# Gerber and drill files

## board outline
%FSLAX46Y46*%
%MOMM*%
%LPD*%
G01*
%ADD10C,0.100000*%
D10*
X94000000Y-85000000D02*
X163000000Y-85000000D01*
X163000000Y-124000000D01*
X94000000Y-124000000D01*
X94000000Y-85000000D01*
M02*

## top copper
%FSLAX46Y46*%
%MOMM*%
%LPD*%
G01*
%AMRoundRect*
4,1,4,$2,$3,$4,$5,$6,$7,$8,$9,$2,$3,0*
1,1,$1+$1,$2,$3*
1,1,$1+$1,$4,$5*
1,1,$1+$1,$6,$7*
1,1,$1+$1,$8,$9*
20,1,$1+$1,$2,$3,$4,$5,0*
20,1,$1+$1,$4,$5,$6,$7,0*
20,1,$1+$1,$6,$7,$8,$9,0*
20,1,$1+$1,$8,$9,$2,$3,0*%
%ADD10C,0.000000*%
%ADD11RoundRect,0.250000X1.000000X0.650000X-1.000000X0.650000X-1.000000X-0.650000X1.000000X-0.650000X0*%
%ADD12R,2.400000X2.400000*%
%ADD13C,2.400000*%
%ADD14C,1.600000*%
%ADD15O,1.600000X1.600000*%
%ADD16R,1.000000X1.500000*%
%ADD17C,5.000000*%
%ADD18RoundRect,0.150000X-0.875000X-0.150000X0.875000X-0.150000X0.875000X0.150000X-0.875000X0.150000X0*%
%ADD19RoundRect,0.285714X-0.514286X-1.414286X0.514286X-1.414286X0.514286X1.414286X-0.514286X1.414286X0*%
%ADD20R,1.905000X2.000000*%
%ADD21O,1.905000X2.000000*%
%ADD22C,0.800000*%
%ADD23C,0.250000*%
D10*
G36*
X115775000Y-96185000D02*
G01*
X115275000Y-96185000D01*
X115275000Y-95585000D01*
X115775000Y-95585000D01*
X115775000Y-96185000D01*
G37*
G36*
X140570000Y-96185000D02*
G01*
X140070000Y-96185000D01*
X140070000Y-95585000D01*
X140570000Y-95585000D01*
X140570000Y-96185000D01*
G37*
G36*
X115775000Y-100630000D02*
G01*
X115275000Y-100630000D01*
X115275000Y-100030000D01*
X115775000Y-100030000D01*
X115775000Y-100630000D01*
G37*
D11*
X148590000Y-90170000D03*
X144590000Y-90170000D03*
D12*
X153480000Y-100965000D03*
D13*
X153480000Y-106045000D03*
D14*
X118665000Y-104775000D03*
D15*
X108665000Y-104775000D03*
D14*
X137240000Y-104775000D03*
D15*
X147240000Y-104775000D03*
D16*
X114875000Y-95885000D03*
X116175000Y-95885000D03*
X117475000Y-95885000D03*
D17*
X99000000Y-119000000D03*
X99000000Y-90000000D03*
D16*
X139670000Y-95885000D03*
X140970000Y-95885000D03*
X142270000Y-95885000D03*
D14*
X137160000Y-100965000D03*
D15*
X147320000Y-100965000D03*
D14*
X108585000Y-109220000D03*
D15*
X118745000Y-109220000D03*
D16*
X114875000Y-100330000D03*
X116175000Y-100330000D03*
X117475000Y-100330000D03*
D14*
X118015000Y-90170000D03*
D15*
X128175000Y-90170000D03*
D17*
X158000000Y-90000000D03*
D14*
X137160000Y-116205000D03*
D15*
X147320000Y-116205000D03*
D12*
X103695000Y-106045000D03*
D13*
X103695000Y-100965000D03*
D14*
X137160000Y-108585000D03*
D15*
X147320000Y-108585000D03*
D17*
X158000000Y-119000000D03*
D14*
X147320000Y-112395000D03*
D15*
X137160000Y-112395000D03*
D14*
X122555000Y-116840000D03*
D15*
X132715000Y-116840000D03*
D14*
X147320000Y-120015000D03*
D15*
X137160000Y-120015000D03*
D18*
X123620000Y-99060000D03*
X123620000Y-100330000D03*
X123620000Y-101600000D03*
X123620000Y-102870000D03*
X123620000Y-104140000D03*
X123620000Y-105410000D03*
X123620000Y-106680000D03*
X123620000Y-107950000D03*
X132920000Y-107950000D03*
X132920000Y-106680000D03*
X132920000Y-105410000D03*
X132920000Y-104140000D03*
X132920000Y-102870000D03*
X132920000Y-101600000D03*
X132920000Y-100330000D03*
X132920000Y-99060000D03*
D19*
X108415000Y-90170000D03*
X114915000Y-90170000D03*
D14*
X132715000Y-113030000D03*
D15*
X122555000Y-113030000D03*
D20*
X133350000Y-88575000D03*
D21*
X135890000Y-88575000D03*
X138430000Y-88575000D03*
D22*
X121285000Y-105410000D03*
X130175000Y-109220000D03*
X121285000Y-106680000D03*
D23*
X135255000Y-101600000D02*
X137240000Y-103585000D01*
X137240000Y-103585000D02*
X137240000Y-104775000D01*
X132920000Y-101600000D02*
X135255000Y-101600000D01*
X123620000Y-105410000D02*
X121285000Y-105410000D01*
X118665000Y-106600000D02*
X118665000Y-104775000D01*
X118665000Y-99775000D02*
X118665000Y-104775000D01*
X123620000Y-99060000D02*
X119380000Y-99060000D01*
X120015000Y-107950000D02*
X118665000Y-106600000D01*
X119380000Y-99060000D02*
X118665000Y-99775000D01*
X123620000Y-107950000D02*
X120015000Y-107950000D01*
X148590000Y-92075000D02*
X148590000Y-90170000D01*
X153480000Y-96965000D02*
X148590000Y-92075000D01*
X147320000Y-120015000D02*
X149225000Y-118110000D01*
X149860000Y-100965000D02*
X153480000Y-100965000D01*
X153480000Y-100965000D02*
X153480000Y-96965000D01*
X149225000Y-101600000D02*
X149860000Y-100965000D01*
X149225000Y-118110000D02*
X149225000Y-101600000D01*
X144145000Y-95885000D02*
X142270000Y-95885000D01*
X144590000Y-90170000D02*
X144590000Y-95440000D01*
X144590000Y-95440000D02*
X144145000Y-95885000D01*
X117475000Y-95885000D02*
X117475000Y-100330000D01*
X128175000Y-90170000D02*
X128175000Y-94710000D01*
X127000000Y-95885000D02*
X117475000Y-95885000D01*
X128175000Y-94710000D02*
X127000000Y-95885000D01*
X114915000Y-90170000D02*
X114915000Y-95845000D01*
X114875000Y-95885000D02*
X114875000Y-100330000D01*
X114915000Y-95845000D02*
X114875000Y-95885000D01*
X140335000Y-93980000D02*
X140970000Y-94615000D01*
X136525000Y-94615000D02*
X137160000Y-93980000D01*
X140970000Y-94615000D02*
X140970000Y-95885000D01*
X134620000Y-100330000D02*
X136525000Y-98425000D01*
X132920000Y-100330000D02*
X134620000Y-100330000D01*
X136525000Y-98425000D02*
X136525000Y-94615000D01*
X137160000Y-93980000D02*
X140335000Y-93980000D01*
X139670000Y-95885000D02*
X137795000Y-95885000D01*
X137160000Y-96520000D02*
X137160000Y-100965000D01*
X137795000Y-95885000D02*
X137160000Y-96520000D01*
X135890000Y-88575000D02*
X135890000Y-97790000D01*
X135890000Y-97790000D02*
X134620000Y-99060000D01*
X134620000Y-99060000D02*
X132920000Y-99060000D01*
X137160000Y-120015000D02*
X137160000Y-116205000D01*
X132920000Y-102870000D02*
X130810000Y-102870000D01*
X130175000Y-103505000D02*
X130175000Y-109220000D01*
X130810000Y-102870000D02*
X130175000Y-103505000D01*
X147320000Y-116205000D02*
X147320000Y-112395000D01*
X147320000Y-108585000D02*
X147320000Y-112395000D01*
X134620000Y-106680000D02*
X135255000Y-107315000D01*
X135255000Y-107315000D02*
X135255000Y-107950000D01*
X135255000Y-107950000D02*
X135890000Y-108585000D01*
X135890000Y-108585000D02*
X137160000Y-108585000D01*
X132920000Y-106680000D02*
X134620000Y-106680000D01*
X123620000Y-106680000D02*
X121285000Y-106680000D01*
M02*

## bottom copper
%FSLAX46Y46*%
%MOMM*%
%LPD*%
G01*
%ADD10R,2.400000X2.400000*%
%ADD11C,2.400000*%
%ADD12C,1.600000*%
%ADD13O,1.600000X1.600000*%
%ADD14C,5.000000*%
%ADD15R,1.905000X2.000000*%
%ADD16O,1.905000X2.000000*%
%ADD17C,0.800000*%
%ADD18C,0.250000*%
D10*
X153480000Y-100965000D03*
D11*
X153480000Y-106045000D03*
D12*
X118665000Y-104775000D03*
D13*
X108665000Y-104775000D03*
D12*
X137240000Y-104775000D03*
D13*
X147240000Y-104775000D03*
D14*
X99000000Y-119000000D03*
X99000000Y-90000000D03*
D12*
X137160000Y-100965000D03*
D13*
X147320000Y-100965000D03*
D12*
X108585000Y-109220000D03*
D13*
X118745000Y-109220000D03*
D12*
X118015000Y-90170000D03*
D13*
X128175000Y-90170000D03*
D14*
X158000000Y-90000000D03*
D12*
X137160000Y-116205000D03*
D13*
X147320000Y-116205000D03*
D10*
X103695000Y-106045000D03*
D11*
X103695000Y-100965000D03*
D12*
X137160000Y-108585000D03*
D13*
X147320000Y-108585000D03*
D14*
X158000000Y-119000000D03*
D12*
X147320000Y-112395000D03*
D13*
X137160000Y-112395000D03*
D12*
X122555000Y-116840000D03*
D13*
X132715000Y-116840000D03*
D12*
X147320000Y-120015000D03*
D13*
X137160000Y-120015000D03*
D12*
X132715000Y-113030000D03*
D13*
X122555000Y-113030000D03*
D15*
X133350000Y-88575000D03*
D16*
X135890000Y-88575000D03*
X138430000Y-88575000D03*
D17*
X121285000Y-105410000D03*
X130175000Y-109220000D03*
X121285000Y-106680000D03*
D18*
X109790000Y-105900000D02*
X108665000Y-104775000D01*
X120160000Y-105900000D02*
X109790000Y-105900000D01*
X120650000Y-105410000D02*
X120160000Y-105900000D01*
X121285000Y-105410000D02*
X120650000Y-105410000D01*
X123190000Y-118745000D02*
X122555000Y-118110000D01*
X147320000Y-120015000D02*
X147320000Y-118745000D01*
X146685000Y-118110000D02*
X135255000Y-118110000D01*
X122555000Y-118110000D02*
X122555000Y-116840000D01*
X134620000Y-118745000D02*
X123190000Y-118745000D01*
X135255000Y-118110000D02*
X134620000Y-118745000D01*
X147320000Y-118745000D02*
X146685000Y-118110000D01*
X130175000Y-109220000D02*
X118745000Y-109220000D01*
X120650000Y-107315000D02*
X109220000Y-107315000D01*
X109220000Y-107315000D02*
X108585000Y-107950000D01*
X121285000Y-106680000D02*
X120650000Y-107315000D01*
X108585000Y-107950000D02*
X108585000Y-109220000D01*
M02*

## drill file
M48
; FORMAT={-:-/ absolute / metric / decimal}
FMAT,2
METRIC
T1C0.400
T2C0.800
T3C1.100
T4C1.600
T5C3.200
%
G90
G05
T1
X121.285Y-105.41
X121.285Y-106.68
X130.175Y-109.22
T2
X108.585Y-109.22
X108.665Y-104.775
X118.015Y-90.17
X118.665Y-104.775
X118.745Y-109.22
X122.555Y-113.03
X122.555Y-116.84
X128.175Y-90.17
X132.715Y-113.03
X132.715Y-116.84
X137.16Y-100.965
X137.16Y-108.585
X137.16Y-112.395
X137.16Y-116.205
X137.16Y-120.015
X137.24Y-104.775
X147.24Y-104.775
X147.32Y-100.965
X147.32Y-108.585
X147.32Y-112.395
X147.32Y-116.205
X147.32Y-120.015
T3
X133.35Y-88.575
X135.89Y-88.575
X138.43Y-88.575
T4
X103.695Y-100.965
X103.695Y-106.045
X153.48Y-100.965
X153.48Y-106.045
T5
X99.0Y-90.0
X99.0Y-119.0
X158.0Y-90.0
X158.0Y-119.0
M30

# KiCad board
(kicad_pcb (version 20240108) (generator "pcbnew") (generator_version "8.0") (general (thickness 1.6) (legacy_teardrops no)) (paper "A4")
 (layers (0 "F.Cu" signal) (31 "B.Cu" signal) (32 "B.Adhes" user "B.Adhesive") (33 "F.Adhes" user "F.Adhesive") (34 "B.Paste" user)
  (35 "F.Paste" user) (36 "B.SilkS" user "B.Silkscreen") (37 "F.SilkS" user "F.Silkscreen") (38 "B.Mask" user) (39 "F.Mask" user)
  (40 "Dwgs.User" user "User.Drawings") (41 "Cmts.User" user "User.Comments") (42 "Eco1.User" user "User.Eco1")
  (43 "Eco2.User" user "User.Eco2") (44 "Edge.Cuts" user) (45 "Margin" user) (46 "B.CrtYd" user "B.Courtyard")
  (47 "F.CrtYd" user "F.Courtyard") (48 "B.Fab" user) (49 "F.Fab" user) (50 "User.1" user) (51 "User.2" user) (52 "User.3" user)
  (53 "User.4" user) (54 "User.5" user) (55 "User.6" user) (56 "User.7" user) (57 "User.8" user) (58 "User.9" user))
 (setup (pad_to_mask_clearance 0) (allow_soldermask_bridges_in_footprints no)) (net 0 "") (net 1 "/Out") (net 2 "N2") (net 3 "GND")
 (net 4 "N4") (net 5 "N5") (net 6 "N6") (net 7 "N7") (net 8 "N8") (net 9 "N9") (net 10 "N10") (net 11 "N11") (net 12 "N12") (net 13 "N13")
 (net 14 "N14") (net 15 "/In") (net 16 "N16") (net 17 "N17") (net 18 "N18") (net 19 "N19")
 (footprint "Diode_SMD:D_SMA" (layer "F.Cu") (at 146.59 90.17 180)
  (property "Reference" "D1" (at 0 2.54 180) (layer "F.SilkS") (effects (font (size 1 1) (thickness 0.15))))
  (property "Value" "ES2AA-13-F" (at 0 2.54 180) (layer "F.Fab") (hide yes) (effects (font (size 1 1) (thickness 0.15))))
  (pad "1" smd roundrect (at -2 0 180) (size 2.5 1.8) (layers "F.Cu" "F.Paste" "F.Mask") (roundrect_rratio 0.1388888889) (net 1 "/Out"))
  (pad "2" smd roundrect (at 2 0 180) (size 2.5 1.8) (layers "F.Cu" "F.Paste" "F.Mask") (roundrect_rratio 0.1388888889) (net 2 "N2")))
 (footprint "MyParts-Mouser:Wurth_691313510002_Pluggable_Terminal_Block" (layer "F.Cu") (at 153.48 100.965 -90)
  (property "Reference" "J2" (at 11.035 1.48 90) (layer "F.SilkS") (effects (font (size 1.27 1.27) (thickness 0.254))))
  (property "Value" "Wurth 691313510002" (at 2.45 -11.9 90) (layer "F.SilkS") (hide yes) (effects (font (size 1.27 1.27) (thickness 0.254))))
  (pad "1" thru_hole rect (at 0 0 270) (size 2.4 2.4) (drill 1.6) (layers "*.Cu" "*.Mask") (remove_unused_layers no) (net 1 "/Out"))
  (pad "2" thru_hole circle (at 5.08 0 270) (size 2.4 2.4) (drill 1.6) (layers "*.Cu" "*.Mask") (remove_unused_layers no) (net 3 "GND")))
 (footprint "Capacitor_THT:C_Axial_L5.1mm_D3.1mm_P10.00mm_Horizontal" (layer "F.Cu") (at 118.665 104.775 180)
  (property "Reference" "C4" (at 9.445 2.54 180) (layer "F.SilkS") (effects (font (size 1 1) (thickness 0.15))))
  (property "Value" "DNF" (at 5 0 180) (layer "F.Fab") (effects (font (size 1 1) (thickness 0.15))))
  (pad "1" thru_hole circle (at 0 0 180) (size 1.6 1.6) (drill 0.8) (layers "*.Cu" "*.Mask") (remove_unused_layers no) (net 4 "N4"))
  (pad "2" thru_hole oval (at 10 0 180) (size 1.6 1.6) (drill 0.8) (layers "*.Cu" "*.Mask") (remove_unused_layers no) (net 3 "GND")))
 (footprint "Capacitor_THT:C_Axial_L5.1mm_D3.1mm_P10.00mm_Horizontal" (layer "F.Cu") (at 137.24 104.775)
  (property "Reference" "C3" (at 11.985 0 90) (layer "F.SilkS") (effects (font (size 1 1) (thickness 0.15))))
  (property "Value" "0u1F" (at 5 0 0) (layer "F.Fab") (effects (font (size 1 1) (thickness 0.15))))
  (pad "1" thru_hole circle (at 0 0) (size 1.6 1.6) (drill 0.8) (layers "*.Cu" "*.Mask") (remove_unused_layers no) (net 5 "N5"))
  (pad "2" thru_hole oval (at 10 0) (size 1.6 1.6) (drill 0.8) (layers "*.Cu" "*.Mask") (remove_unused_layers no) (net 3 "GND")))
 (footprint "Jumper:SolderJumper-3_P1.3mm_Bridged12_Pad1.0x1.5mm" (layer "F.Cu") (at 116.175 95.885)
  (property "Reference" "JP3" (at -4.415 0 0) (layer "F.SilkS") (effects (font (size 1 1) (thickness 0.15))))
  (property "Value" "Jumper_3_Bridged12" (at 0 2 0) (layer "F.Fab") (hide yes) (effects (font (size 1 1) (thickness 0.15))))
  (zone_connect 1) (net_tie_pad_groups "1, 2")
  (fp_poly (pts (xy -0.9 -0.3) (xy -0.4 -0.3) (xy -0.4 0.3) (xy -0.9 0.3)) (stroke (width 0) (type solid)) (fill solid) (layer "F.Cu"))
  (pad "1" smd rect (at -1.3 0) (size 1 1.5) (layers "F.Cu" "F.Mask") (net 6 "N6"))
  (pad "2" smd rect (at 0 0) (size 1 1.5) (layers "F.Cu" "F.Mask") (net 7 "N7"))
  (pad "3" smd rect (at 1.3 0) (size 1 1.5) (layers "F.Cu" "F.Mask") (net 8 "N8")))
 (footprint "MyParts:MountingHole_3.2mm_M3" (layer "F.Cu") (at 99 119)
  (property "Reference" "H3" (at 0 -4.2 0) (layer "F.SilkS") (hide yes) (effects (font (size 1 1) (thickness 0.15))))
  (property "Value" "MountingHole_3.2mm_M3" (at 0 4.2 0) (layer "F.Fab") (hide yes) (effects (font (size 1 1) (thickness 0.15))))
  (pad "" np_thru_hole circle (at 0 0) (size 5 5) (drill 3.2) (layers "*.Cu" "*.Mask")))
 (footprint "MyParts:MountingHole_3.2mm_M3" (layer "F.Cu") (at 99 90)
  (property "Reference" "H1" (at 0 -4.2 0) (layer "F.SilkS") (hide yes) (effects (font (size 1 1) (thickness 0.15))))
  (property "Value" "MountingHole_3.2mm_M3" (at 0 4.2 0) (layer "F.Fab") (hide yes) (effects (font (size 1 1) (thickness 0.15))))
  (pad "" np_thru_hole circle (at 0 0) (size 5 5) (drill 3.2) (layers "*.Cu" "*.Mask")))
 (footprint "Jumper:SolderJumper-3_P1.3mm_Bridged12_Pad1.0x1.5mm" (layer "F.Cu") (at 140.97 95.885)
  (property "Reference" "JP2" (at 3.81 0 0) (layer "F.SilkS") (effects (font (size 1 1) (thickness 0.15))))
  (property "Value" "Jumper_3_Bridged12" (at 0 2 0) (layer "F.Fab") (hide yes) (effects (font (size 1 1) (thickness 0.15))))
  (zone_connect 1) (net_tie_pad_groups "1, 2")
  (fp_poly (pts (xy -0.9 -0.3) (xy -0.4 -0.3) (xy -0.4 0.3) (xy -0.9 0.3)) (stroke (width 0) (type solid)) (fill solid) (layer "F.Cu"))
  (pad "1" smd rect (at -1.3 0) (size 1 1.5) (layers "F.Cu" "F.Mask") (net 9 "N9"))
  (pad "2" smd rect (at 0 0) (size 1 1.5) (layers "F.Cu" "F.Mask") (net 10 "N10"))
  (pad "3" smd rect (at 1.3 0) (size 1 1.5) (layers "F.Cu" "F.Mask") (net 2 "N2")))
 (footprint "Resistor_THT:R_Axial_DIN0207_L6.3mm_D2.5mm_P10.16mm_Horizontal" (layer "F.Cu") (at 137.16 100.965)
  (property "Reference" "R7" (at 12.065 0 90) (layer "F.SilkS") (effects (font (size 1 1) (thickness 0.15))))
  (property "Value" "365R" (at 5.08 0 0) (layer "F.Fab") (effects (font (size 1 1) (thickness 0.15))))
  (pad "1" thru_hole circle (at 0 0) (size 1.6 1.6) (drill 0.8) (layers "*.Cu" "*.Mask") (remove_unused_layers no) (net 9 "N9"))
  (pad "2" thru_hole oval (at 10.16 0) (size 1.6 1.6) (drill 0.8) (layers "*.Cu" "*.Mask") (remove_unused_layers no) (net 3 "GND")))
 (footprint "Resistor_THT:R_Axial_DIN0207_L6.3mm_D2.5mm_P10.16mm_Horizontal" (layer "F.Cu") (at 108.585 109.22)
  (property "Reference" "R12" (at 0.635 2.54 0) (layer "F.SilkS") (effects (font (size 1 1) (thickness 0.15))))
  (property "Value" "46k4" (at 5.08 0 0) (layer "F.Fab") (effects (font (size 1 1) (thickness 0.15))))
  (pad "1" thru_hole circle (at 0 0) (size 1.6 1.6) (drill 0.8) (layers "*.Cu" "*.Mask") (remove_unused_layers no) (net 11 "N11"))
  (pad "2" thru_hole oval (at 10.16 0) (size 1.6 1.6) (drill 0.8) (layers "*.Cu" "*.Mask") (remove_unused_layers no) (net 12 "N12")))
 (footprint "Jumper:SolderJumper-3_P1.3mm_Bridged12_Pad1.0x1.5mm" (layer "F.Cu") (at 116.175 100.33)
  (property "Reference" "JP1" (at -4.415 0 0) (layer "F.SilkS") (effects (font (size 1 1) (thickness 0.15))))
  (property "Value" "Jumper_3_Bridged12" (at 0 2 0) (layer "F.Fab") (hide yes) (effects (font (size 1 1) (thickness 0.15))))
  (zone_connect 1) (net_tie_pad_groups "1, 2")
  (fp_poly (pts (xy -0.9 -0.3) (xy -0.4 -0.3) (xy -0.4 0.3) (xy -0.9 0.3)) (stroke (width 0) (type solid)) (fill solid) (layer "F.Cu"))
  (pad "1" smd rect (at -1.3 0) (size 1 1.5) (layers "F.Cu" "F.Mask") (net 6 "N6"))
  (pad "2" smd rect (at 0 0) (size 1 1.5) (layers "F.Cu" "F.Mask") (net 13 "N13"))
  (pad "3" smd rect (at 1.3 0) (size 1 1.5) (layers "F.Cu" "F.Mask") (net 8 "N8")))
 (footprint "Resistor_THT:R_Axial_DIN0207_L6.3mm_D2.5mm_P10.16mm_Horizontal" (layer "F.Cu") (at 118.015 90.17)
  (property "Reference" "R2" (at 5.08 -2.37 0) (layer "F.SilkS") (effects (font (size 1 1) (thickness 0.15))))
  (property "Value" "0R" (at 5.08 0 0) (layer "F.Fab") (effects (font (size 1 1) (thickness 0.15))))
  (pad "1" thru_hole circle (at 0 0) (size 1.6 1.6) (drill 0.8) (layers "*.Cu" "*.Mask") (remove_unused_layers no) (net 6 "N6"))
  (pad "2" thru_hole oval (at 10.16 0) (size 1.6 1.6) (drill 0.8) (layers "*.Cu" "*.Mask") (remove_unused_layers no) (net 8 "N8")))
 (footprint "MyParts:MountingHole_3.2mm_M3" (layer "F.Cu") (at 158 90)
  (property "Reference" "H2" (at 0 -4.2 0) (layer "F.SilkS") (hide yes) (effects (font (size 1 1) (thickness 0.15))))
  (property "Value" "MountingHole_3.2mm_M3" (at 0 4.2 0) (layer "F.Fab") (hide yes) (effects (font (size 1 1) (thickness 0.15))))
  (pad "" np_thru_hole circle (at 0 0) (size 5 5) (drill 3.2) (layers "*.Cu" "*.Mask")))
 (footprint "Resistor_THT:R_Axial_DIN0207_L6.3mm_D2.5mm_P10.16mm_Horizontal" (layer "F.Cu") (at 137.16 116.205)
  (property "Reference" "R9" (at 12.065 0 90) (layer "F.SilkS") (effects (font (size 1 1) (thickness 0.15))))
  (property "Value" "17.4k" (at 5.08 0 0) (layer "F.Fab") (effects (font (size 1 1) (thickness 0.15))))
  (pad "1" thru_hole circle (at 0 0) (size 1.6 1.6) (drill 0.8) (layers "*.Cu" "*.Mask") (remove_unused_layers no) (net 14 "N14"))
  (pad "2" thru_hole oval (at 10.16 0) (size 1.6 1.6) (drill 0.8) (layers "*.Cu" "*.Mask") (remove_unused_layers no) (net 12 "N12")))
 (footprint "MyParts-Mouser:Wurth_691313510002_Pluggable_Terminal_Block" (layer "F.Cu") (at 103.695 106.045 90)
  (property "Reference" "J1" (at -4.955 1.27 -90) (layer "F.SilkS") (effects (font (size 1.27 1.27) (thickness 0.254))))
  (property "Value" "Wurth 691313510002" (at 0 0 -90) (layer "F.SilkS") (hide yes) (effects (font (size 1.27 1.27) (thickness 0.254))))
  (pad "1" thru_hole rect (at 0 0 90) (size 2.4 2.4) (drill 1.6) (layers "*.Cu" "*.Mask") (remove_unused_layers no) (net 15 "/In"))
  (pad "2" thru_hole circle (at 5.08 0 90) (size 2.4 2.4) (drill 1.6) (layers "*.Cu" "*.Mask") (remove_unused_layers no) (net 3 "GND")))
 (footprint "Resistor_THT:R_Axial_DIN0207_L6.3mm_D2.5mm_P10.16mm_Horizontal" (layer "F.Cu") (at 137.16 108.585)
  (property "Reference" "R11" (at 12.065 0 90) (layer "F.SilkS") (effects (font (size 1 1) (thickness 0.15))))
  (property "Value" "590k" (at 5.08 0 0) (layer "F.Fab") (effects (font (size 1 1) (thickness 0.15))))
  (pad "1" thru_hole circle (at 0 0) (size 1.6 1.6) (drill 0.8) (layers "*.Cu" "*.Mask") (remove_unused_layers no) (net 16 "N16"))
  (pad "2" thru_hole oval (at 10.16 0) (size 1.6 1.6) (drill 0.8) (layers "*.Cu" "*.Mask") (remove_unused_layers no) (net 12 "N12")))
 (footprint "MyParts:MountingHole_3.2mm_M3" (layer "F.Cu") (at 158 119)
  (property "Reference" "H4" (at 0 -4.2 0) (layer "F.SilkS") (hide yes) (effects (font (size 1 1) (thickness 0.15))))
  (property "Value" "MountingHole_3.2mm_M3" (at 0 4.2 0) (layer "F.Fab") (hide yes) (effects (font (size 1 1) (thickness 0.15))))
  (pad "" np_thru_hole circle (at 0 0) (size 5 5) (drill 3.2) (layers "*.Cu" "*.Mask")))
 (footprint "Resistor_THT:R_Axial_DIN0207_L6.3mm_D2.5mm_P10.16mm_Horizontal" (layer "F.Cu") (at 147.32 112.395 180)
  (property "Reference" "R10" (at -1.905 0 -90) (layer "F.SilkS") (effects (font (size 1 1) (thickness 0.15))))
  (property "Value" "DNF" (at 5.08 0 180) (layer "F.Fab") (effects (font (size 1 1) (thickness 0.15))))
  (pad "1" thru_hole circle (at 0 0 180) (size 1.6 1.6) (drill 0.8) (layers "*.Cu" "*.Mask") (remove_unused_layers no) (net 12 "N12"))
  (pad "2" thru_hole oval (at 10.16 0 180) (size 1.6 1.6) (drill 0.8) (layers "*.Cu" "*.Mask") (remove_unused_layers no) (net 3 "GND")))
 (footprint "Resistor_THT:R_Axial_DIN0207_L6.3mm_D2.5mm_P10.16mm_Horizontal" (layer "F.Cu") (at 122.555 116.84)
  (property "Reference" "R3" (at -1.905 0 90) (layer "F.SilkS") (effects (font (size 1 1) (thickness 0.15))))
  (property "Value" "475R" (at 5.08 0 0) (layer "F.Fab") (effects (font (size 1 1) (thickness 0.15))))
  (pad "1" thru_hole circle (at 0 0) (size 1.6 1.6) (drill 0.8) (layers "*.Cu" "*.Mask") (remove_unused_layers no) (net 1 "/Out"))
  (pad "2" thru_hole oval (at 10.16 0) (size 1.6 1.6) (drill 0.8) (layers "*.Cu" "*.Mask") (remove_unused_layers no) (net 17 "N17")))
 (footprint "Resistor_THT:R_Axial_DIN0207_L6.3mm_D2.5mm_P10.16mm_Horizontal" (layer "F.Cu") (at 147.32 120.015 180)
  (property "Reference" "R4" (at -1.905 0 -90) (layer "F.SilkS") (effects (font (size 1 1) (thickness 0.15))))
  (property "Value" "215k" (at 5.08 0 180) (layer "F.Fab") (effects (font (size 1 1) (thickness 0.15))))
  (pad "1" thru_hole circle (at 0 0 180) (size 1.6 1.6) (drill 0.8) (layers "*.Cu" "*.Mask") (remove_unused_layers no) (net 1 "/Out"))
  (pad "2" thru_hole oval (at 10.16 0 180) (size 1.6 1.6) (drill 0.8) (layers "*.Cu" "*.Mask") (remove_unused_layers no) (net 14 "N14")))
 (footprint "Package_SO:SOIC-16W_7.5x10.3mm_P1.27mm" (layer "F.Cu") (at 128.27 103.505)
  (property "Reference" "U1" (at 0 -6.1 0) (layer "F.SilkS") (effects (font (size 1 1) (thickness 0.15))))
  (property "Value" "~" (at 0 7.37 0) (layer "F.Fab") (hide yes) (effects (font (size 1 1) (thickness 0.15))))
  (pad "1" smd roundrect (at -4.65 -4.445) (size 2.05 0.6) (layers "F.Cu" "F.Paste" "F.Mask") (roundrect_rratio 0.25) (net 4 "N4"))
  (pad "2" smd roundrect (at -4.65 -3.175) (size 2.05 0.6) (layers "F.Cu" "F.Paste" "F.Mask") (roundrect_rratio 0.25) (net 13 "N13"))
  (pad "3" smd roundrect (at -4.65 -1.905) (size 2.05 0.6) (layers "F.Cu" "F.Paste" "F.Mask") (roundrect_rratio 0.25) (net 15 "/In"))
  (pad "4" smd roundrect (at -4.65 -0.635) (size 2.05 0.6) (layers "F.Cu" "F.Paste" "F.Mask") (roundrect_rratio 0.25) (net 7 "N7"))
  (pad "5" smd roundrect (at -4.65 0.635) (size 2.05 0.6) (layers "F.Cu" "F.Paste" "F.Mask") (roundrect_rratio 0.25) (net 15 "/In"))
  (pad "6" smd roundrect (at -4.65 1.905) (size 2.05 0.6) (layers "F.Cu" "F.Paste" "F.Mask") (roundrect_rratio 0.25) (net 3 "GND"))
  (pad "7" smd roundrect (at -4.65 3.175) (size 2.05 0.6) (layers "F.Cu" "F.Paste" "F.Mask") (roundrect_rratio 0.25) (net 11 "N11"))
  (pad "8" smd roundrect (at -4.65 4.445) (size 2.05 0.6) (layers "F.Cu" "F.Paste" "F.Mask") (roundrect_rratio 0.25) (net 4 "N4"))
  (pad "9" smd roundrect (at 4.65 4.445) (size 2.05 0.6) (layers "F.Cu" "F.Paste" "F.Mask") (roundrect_rratio 0.25) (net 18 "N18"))
  (pad "10" smd roundrect (at 4.65 3.175) (size 2.05 0.6) (layers "F.Cu" "F.Paste" "F.Mask") (roundrect_rratio 0.25) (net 16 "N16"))
  (pad "11" smd roundrect (at 4.65 1.905) (size 2.05 0.6) (layers "F.Cu" "F.Paste" "F.Mask") (roundrect_rratio 0.25) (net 17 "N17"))
  (pad "12" smd roundrect (at 4.65 0.635) (size 2.05 0.6) (layers "F.Cu" "F.Paste" "F.Mask") (roundrect_rratio 0.25) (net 14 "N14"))
  (pad "13" smd roundrect (at 4.65 -0.635) (size 2.05 0.6) (layers "F.Cu" "F.Paste" "F.Mask") (roundrect_rratio 0.25) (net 12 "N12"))
  (pad "14" smd roundrect (at 4.65 -1.905) (size 2.05 0.6) (layers "F.Cu" "F.Paste" "F.Mask") (roundrect_rratio 0.25) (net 5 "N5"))
  (pad "15" smd roundrect (at 4.65 -3.175) (size 2.05 0.6) (layers "F.Cu" "F.Paste" "F.Mask") (roundrect_rratio 0.25) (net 10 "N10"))
  (pad "16" smd roundrect (at 4.65 -4.445) (size 2.05 0.6) (layers "F.Cu" "F.Paste" "F.Mask") (roundrect_rratio 0.25) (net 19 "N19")))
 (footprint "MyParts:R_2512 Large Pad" (layer "F.Cu") (at 111.665 90.17)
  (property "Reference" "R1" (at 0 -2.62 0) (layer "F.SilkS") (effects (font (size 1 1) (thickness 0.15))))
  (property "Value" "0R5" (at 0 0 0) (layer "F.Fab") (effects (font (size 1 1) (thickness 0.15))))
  (pad "1" smd roundrect (at -3.25 0) (size 1.6 3.4) (layers "F.Cu" "F.Paste" "F.Mask") (roundrect_rratio 0.178571) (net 15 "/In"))
  (pad "2" smd roundrect (at 3.25 0) (size 1.6 3.4) (layers "F.Cu" "F.Paste" "F.Mask") (roundrect_rratio 0.178571) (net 6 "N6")))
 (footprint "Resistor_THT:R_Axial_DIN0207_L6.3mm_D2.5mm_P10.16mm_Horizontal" (layer "F.Cu") (at 132.715 113.03 180)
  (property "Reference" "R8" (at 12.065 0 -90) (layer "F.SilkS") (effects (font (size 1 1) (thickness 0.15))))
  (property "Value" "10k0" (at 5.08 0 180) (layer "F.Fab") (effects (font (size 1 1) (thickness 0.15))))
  (pad "1" thru_hole circle (at 0 0 180) (size 1.6 1.6) (drill 0.8) (layers "*.Cu" "*.Mask") (remove_unused_layers no) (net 18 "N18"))
  (pad "2" thru_hole oval (at 10.16 0 180) (size 1.6 1.6) (drill 0.8) (layers "*.Cu" "*.Mask") (remove_unused_layers no) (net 1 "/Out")))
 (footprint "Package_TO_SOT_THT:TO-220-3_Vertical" (layer "F.Cu") (at 133.35 88.575)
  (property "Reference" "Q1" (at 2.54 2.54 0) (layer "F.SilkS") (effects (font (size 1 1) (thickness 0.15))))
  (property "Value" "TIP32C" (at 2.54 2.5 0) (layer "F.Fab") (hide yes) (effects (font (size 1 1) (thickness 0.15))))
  (pad "1" thru_hole rect (at 0 0) (size 1.905 2) (drill 1.1) (layers "*.Cu" "*.Mask") (remove_unused_layers no) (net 2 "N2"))
  (pad "2" thru_hole oval (at 2.54 0) (size 1.905 2) (drill 1.1) (layers "*.Cu" "*.Mask") (remove_unused_layers no) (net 19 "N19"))
  (pad "3" thru_hole oval (at 5.08 0) (size 1.905 2) (drill 1.1) (layers "*.Cu" "*.Mask") (remove_unused_layers no) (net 8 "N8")))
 (gr_rect (start 94 85) (end 163 124) (stroke (width 0.1) (type default)) (fill none) (layer "Edge.Cuts"))
 (segment (start 135.255 101.6) (end 137.24 103.585) (width 0.25) (layer "F.Cu") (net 5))
 (segment (start 137.24 103.585) (end 137.24 104.775) (width 0.25) (layer "F.Cu") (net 5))
 (segment (start 132.92 101.6) (end 135.255 101.6) (width 0.25) (layer "F.Cu") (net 5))
 (segment (start 123.62 105.41) (end 121.285 105.41) (width 0.25) (layer "F.Cu") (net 3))
 (via (at 121.285 105.41) (size 0.8) (drill 0.4) (layers "F.Cu" "B.Cu") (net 3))
 (segment (start 109.79 105.9) (end 108.665 104.775) (width 0.25) (layer "B.Cu") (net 3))
 (segment (start 120.16 105.9) (end 109.79 105.9) (width 0.25) (layer "B.Cu") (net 3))
 (segment (start 120.65 105.41) (end 120.16 105.9) (width 0.25) (layer "B.Cu") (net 3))
 (segment (start 121.285 105.41) (end 120.65 105.41) (width 0.25) (layer "B.Cu") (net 3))
 (segment (start 118.665 106.6) (end 118.665 104.775) (width 0.25) (layer "F.Cu") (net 4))
 (segment (start 118.665 99.775) (end 118.665 104.775) (width 0.25) (layer "F.Cu") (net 4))
 (segment (start 123.62 99.06) (end 119.38 99.06) (width 0.25) (layer "F.Cu") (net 4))
 (segment (start 120.015 107.95) (end 118.665 106.6) (width 0.25) (layer "F.Cu") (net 4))
 (segment (start 119.38 99.06) (end 118.665 99.775) (width 0.25) (layer "F.Cu") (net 4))
 (segment (start 123.62 107.95) (end 120.015 107.95) (width 0.25) (layer "F.Cu") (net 4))
 (segment (start 148.59 92.075) (end 148.59 90.17) (width 0.25) (layer "F.Cu") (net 1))
 (segment (start 153.48 96.965) (end 148.59 92.075) (width 0.25) (layer "F.Cu") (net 1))
 (segment (start 147.32 120.015) (end 149.225 118.11) (width 0.25) (layer "F.Cu") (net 1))
 (segment (start 149.86 100.965) (end 153.48 100.965) (width 0.25) (layer "F.Cu") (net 1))
 (segment (start 153.48 100.965) (end 153.48 96.965) (width 0.25) (layer "F.Cu") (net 1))
 (segment (start 149.225 101.6) (end 149.86 100.965) (width 0.25) (layer "F.Cu") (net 1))
 (segment (start 149.225 118.11) (end 149.225 101.6) (width 0.25) (layer "F.Cu") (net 1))
 (segment (start 123.19 118.745) (end 122.555 118.11) (width 0.25) (layer "B.Cu") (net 1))
 (segment (start 147.32 120.015) (end 147.32 118.745) (width 0.25) (layer "B.Cu") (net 1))
 (segment (start 146.685 118.11) (end 135.255 118.11) (width 0.25) (layer "B.Cu") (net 1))
 (segment (start 122.555 118.11) (end 122.555 116.84) (width 0.25) (layer "B.Cu") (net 1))
 (segment (start 134.62 118.745) (end 123.19 118.745) (width 0.25) (layer "B.Cu") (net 1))
 (segment (start 135.255 118.11) (end 134.62 118.745) (width 0.25) (layer "B.Cu") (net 1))
 (segment (start 147.32 118.745) (end 146.685 118.11) (width 0.25) (layer "B.Cu") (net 1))
 (segment (start 144.145 95.885) (end 142.27 95.885) (width 0.25) (layer "F.Cu") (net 2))
 (segment (start 144.59 90.17) (end 144.59 95.44) (width 0.25) (layer "F.Cu") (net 2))
 (segment (start 144.59 95.44) (end 144.145 95.885) (width 0.25) (layer "F.Cu") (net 2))
 (segment (start 117.475 95.885) (end 117.475 100.33) (width 0.25) (layer "F.Cu") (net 8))
 (segment (start 128.175 90.17) (end 128.175 94.71) (width 0.25) (layer "F.Cu") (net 8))
 (segment (start 127 95.885) (end 117.475 95.885) (width 0.25) (layer "F.Cu") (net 8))
 (segment (start 128.175 94.71) (end 127 95.885) (width 0.25) (layer "F.Cu") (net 8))
 (segment (start 114.915 90.17) (end 114.915 95.845) (width 0.25) (layer "F.Cu") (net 6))
 (segment (start 114.875 95.885) (end 114.875 100.33) (width 0.25) (layer "F.Cu") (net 6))
 (segment (start 114.915 95.845) (end 114.875 95.885) (width 0.25) (layer "F.Cu") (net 6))
 (segment (start 140.335 93.98) (end 140.97 94.615) (width 0.25) (layer "F.Cu") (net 10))
 (segment (start 136.525 94.615) (end 137.16 93.98) (width 0.25) (layer "F.Cu") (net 10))
 (segment (start 140.97 94.615) (end 140.97 95.885) (width 0.25) (layer "F.Cu") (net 10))
 (segment (start 134.62 100.33) (end 136.525 98.425) (width 0.25) (layer "F.Cu") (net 10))
 (segment (start 132.92 100.33) (end 134.62 100.33) (width 0.25) (layer "F.Cu") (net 10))
 (segment (start 136.525 98.425) (end 136.525 94.615) (width 0.25) (layer "F.Cu") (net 10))
 (segment (start 137.16 93.98) (end 140.335 93.98) (width 0.25) (layer "F.Cu") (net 10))
 (segment (start 139.67 95.885) (end 137.795 95.885) (width 0.25) (layer "F.Cu") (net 9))
 (segment (start 137.16 96.52) (end 137.16 100.965) (width 0.25) (layer "F.Cu") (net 9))
 (segment (start 137.795 95.885) (end 137.16 96.52) (width 0.25) (layer "F.Cu") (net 9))
 (segment (start 135.89 88.575) (end 135.89 97.79) (width 0.25) (layer "F.Cu") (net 19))
 (segment (start 135.89 97.79) (end 134.62 99.06) (width 0.25) (layer "F.Cu") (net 19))
 (segment (start 134.62 99.06) (end 132.92 99.06) (width 0.25) (layer "F.Cu") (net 19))
 (segment (start 137.16 120.015) (end 137.16 116.205) (width 0.25) (layer "F.Cu") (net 14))
 (segment (start 132.92 102.87) (end 130.81 102.87) (width 0.25) (layer "F.Cu") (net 12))
 (segment (start 130.175 103.505) (end 130.175 109.22) (width 0.25) (layer "F.Cu") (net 12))
 (segment (start 130.81 102.87) (end 130.175 103.505) (width 0.25) (layer "F.Cu") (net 12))
 (segment (start 147.32 116.205) (end 147.32 112.395) (width 0.25) (layer "F.Cu") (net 12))
 (segment (start 147.32 108.585) (end 147.32 112.395) (width 0.25) (layer "F.Cu") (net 12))
 (via (at 130.175 109.22) (size 0.8) (drill 0.4) (layers "F.Cu" "B.Cu") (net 12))
 (segment (start 130.175 109.22) (end 118.745 109.22) (width 0.25) (layer "B.Cu") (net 12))
 (segment (start 134.62 106.68) (end 135.255 107.315) (width 0.25) (layer "F.Cu") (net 16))
 (segment (start 135.255 107.315) (end 135.255 107.95) (width 0.25) (layer "F.Cu") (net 16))
 (segment (start 135.255 107.95) (end 135.89 108.585) (width 0.25) (layer "F.Cu") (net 16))
 (segment (start 135.89 108.585) (end 137.16 108.585) (width 0.25) (layer "F.Cu") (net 16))
 (segment (start 132.92 106.68) (end 134.62 106.68) (width 0.25) (layer "F.Cu") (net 16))
 (segment (start 123.62 106.68) (end 121.285 106.68) (width 0.25) (layer "F.Cu") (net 11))
 (via (at 121.285 106.68) (size 0.8) (drill 0.4) (layers "F.Cu" "B.Cu") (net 11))
 (segment (start 120.65 107.315) (end 109.22 107.315) (width 0.25) (layer "B.Cu") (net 11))
 (segment (start 109.22 107.315) (end 108.585 107.95) (width 0.25) (layer "B.Cu") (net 11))
 (segment (start 121.285 106.68) (end 120.65 107.315) (width 0.25) (layer "B.Cu") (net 11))
 (segment (start 108.585 107.95) (end 108.585 109.22) (width 0.25) (layer "B.Cu") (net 11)))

